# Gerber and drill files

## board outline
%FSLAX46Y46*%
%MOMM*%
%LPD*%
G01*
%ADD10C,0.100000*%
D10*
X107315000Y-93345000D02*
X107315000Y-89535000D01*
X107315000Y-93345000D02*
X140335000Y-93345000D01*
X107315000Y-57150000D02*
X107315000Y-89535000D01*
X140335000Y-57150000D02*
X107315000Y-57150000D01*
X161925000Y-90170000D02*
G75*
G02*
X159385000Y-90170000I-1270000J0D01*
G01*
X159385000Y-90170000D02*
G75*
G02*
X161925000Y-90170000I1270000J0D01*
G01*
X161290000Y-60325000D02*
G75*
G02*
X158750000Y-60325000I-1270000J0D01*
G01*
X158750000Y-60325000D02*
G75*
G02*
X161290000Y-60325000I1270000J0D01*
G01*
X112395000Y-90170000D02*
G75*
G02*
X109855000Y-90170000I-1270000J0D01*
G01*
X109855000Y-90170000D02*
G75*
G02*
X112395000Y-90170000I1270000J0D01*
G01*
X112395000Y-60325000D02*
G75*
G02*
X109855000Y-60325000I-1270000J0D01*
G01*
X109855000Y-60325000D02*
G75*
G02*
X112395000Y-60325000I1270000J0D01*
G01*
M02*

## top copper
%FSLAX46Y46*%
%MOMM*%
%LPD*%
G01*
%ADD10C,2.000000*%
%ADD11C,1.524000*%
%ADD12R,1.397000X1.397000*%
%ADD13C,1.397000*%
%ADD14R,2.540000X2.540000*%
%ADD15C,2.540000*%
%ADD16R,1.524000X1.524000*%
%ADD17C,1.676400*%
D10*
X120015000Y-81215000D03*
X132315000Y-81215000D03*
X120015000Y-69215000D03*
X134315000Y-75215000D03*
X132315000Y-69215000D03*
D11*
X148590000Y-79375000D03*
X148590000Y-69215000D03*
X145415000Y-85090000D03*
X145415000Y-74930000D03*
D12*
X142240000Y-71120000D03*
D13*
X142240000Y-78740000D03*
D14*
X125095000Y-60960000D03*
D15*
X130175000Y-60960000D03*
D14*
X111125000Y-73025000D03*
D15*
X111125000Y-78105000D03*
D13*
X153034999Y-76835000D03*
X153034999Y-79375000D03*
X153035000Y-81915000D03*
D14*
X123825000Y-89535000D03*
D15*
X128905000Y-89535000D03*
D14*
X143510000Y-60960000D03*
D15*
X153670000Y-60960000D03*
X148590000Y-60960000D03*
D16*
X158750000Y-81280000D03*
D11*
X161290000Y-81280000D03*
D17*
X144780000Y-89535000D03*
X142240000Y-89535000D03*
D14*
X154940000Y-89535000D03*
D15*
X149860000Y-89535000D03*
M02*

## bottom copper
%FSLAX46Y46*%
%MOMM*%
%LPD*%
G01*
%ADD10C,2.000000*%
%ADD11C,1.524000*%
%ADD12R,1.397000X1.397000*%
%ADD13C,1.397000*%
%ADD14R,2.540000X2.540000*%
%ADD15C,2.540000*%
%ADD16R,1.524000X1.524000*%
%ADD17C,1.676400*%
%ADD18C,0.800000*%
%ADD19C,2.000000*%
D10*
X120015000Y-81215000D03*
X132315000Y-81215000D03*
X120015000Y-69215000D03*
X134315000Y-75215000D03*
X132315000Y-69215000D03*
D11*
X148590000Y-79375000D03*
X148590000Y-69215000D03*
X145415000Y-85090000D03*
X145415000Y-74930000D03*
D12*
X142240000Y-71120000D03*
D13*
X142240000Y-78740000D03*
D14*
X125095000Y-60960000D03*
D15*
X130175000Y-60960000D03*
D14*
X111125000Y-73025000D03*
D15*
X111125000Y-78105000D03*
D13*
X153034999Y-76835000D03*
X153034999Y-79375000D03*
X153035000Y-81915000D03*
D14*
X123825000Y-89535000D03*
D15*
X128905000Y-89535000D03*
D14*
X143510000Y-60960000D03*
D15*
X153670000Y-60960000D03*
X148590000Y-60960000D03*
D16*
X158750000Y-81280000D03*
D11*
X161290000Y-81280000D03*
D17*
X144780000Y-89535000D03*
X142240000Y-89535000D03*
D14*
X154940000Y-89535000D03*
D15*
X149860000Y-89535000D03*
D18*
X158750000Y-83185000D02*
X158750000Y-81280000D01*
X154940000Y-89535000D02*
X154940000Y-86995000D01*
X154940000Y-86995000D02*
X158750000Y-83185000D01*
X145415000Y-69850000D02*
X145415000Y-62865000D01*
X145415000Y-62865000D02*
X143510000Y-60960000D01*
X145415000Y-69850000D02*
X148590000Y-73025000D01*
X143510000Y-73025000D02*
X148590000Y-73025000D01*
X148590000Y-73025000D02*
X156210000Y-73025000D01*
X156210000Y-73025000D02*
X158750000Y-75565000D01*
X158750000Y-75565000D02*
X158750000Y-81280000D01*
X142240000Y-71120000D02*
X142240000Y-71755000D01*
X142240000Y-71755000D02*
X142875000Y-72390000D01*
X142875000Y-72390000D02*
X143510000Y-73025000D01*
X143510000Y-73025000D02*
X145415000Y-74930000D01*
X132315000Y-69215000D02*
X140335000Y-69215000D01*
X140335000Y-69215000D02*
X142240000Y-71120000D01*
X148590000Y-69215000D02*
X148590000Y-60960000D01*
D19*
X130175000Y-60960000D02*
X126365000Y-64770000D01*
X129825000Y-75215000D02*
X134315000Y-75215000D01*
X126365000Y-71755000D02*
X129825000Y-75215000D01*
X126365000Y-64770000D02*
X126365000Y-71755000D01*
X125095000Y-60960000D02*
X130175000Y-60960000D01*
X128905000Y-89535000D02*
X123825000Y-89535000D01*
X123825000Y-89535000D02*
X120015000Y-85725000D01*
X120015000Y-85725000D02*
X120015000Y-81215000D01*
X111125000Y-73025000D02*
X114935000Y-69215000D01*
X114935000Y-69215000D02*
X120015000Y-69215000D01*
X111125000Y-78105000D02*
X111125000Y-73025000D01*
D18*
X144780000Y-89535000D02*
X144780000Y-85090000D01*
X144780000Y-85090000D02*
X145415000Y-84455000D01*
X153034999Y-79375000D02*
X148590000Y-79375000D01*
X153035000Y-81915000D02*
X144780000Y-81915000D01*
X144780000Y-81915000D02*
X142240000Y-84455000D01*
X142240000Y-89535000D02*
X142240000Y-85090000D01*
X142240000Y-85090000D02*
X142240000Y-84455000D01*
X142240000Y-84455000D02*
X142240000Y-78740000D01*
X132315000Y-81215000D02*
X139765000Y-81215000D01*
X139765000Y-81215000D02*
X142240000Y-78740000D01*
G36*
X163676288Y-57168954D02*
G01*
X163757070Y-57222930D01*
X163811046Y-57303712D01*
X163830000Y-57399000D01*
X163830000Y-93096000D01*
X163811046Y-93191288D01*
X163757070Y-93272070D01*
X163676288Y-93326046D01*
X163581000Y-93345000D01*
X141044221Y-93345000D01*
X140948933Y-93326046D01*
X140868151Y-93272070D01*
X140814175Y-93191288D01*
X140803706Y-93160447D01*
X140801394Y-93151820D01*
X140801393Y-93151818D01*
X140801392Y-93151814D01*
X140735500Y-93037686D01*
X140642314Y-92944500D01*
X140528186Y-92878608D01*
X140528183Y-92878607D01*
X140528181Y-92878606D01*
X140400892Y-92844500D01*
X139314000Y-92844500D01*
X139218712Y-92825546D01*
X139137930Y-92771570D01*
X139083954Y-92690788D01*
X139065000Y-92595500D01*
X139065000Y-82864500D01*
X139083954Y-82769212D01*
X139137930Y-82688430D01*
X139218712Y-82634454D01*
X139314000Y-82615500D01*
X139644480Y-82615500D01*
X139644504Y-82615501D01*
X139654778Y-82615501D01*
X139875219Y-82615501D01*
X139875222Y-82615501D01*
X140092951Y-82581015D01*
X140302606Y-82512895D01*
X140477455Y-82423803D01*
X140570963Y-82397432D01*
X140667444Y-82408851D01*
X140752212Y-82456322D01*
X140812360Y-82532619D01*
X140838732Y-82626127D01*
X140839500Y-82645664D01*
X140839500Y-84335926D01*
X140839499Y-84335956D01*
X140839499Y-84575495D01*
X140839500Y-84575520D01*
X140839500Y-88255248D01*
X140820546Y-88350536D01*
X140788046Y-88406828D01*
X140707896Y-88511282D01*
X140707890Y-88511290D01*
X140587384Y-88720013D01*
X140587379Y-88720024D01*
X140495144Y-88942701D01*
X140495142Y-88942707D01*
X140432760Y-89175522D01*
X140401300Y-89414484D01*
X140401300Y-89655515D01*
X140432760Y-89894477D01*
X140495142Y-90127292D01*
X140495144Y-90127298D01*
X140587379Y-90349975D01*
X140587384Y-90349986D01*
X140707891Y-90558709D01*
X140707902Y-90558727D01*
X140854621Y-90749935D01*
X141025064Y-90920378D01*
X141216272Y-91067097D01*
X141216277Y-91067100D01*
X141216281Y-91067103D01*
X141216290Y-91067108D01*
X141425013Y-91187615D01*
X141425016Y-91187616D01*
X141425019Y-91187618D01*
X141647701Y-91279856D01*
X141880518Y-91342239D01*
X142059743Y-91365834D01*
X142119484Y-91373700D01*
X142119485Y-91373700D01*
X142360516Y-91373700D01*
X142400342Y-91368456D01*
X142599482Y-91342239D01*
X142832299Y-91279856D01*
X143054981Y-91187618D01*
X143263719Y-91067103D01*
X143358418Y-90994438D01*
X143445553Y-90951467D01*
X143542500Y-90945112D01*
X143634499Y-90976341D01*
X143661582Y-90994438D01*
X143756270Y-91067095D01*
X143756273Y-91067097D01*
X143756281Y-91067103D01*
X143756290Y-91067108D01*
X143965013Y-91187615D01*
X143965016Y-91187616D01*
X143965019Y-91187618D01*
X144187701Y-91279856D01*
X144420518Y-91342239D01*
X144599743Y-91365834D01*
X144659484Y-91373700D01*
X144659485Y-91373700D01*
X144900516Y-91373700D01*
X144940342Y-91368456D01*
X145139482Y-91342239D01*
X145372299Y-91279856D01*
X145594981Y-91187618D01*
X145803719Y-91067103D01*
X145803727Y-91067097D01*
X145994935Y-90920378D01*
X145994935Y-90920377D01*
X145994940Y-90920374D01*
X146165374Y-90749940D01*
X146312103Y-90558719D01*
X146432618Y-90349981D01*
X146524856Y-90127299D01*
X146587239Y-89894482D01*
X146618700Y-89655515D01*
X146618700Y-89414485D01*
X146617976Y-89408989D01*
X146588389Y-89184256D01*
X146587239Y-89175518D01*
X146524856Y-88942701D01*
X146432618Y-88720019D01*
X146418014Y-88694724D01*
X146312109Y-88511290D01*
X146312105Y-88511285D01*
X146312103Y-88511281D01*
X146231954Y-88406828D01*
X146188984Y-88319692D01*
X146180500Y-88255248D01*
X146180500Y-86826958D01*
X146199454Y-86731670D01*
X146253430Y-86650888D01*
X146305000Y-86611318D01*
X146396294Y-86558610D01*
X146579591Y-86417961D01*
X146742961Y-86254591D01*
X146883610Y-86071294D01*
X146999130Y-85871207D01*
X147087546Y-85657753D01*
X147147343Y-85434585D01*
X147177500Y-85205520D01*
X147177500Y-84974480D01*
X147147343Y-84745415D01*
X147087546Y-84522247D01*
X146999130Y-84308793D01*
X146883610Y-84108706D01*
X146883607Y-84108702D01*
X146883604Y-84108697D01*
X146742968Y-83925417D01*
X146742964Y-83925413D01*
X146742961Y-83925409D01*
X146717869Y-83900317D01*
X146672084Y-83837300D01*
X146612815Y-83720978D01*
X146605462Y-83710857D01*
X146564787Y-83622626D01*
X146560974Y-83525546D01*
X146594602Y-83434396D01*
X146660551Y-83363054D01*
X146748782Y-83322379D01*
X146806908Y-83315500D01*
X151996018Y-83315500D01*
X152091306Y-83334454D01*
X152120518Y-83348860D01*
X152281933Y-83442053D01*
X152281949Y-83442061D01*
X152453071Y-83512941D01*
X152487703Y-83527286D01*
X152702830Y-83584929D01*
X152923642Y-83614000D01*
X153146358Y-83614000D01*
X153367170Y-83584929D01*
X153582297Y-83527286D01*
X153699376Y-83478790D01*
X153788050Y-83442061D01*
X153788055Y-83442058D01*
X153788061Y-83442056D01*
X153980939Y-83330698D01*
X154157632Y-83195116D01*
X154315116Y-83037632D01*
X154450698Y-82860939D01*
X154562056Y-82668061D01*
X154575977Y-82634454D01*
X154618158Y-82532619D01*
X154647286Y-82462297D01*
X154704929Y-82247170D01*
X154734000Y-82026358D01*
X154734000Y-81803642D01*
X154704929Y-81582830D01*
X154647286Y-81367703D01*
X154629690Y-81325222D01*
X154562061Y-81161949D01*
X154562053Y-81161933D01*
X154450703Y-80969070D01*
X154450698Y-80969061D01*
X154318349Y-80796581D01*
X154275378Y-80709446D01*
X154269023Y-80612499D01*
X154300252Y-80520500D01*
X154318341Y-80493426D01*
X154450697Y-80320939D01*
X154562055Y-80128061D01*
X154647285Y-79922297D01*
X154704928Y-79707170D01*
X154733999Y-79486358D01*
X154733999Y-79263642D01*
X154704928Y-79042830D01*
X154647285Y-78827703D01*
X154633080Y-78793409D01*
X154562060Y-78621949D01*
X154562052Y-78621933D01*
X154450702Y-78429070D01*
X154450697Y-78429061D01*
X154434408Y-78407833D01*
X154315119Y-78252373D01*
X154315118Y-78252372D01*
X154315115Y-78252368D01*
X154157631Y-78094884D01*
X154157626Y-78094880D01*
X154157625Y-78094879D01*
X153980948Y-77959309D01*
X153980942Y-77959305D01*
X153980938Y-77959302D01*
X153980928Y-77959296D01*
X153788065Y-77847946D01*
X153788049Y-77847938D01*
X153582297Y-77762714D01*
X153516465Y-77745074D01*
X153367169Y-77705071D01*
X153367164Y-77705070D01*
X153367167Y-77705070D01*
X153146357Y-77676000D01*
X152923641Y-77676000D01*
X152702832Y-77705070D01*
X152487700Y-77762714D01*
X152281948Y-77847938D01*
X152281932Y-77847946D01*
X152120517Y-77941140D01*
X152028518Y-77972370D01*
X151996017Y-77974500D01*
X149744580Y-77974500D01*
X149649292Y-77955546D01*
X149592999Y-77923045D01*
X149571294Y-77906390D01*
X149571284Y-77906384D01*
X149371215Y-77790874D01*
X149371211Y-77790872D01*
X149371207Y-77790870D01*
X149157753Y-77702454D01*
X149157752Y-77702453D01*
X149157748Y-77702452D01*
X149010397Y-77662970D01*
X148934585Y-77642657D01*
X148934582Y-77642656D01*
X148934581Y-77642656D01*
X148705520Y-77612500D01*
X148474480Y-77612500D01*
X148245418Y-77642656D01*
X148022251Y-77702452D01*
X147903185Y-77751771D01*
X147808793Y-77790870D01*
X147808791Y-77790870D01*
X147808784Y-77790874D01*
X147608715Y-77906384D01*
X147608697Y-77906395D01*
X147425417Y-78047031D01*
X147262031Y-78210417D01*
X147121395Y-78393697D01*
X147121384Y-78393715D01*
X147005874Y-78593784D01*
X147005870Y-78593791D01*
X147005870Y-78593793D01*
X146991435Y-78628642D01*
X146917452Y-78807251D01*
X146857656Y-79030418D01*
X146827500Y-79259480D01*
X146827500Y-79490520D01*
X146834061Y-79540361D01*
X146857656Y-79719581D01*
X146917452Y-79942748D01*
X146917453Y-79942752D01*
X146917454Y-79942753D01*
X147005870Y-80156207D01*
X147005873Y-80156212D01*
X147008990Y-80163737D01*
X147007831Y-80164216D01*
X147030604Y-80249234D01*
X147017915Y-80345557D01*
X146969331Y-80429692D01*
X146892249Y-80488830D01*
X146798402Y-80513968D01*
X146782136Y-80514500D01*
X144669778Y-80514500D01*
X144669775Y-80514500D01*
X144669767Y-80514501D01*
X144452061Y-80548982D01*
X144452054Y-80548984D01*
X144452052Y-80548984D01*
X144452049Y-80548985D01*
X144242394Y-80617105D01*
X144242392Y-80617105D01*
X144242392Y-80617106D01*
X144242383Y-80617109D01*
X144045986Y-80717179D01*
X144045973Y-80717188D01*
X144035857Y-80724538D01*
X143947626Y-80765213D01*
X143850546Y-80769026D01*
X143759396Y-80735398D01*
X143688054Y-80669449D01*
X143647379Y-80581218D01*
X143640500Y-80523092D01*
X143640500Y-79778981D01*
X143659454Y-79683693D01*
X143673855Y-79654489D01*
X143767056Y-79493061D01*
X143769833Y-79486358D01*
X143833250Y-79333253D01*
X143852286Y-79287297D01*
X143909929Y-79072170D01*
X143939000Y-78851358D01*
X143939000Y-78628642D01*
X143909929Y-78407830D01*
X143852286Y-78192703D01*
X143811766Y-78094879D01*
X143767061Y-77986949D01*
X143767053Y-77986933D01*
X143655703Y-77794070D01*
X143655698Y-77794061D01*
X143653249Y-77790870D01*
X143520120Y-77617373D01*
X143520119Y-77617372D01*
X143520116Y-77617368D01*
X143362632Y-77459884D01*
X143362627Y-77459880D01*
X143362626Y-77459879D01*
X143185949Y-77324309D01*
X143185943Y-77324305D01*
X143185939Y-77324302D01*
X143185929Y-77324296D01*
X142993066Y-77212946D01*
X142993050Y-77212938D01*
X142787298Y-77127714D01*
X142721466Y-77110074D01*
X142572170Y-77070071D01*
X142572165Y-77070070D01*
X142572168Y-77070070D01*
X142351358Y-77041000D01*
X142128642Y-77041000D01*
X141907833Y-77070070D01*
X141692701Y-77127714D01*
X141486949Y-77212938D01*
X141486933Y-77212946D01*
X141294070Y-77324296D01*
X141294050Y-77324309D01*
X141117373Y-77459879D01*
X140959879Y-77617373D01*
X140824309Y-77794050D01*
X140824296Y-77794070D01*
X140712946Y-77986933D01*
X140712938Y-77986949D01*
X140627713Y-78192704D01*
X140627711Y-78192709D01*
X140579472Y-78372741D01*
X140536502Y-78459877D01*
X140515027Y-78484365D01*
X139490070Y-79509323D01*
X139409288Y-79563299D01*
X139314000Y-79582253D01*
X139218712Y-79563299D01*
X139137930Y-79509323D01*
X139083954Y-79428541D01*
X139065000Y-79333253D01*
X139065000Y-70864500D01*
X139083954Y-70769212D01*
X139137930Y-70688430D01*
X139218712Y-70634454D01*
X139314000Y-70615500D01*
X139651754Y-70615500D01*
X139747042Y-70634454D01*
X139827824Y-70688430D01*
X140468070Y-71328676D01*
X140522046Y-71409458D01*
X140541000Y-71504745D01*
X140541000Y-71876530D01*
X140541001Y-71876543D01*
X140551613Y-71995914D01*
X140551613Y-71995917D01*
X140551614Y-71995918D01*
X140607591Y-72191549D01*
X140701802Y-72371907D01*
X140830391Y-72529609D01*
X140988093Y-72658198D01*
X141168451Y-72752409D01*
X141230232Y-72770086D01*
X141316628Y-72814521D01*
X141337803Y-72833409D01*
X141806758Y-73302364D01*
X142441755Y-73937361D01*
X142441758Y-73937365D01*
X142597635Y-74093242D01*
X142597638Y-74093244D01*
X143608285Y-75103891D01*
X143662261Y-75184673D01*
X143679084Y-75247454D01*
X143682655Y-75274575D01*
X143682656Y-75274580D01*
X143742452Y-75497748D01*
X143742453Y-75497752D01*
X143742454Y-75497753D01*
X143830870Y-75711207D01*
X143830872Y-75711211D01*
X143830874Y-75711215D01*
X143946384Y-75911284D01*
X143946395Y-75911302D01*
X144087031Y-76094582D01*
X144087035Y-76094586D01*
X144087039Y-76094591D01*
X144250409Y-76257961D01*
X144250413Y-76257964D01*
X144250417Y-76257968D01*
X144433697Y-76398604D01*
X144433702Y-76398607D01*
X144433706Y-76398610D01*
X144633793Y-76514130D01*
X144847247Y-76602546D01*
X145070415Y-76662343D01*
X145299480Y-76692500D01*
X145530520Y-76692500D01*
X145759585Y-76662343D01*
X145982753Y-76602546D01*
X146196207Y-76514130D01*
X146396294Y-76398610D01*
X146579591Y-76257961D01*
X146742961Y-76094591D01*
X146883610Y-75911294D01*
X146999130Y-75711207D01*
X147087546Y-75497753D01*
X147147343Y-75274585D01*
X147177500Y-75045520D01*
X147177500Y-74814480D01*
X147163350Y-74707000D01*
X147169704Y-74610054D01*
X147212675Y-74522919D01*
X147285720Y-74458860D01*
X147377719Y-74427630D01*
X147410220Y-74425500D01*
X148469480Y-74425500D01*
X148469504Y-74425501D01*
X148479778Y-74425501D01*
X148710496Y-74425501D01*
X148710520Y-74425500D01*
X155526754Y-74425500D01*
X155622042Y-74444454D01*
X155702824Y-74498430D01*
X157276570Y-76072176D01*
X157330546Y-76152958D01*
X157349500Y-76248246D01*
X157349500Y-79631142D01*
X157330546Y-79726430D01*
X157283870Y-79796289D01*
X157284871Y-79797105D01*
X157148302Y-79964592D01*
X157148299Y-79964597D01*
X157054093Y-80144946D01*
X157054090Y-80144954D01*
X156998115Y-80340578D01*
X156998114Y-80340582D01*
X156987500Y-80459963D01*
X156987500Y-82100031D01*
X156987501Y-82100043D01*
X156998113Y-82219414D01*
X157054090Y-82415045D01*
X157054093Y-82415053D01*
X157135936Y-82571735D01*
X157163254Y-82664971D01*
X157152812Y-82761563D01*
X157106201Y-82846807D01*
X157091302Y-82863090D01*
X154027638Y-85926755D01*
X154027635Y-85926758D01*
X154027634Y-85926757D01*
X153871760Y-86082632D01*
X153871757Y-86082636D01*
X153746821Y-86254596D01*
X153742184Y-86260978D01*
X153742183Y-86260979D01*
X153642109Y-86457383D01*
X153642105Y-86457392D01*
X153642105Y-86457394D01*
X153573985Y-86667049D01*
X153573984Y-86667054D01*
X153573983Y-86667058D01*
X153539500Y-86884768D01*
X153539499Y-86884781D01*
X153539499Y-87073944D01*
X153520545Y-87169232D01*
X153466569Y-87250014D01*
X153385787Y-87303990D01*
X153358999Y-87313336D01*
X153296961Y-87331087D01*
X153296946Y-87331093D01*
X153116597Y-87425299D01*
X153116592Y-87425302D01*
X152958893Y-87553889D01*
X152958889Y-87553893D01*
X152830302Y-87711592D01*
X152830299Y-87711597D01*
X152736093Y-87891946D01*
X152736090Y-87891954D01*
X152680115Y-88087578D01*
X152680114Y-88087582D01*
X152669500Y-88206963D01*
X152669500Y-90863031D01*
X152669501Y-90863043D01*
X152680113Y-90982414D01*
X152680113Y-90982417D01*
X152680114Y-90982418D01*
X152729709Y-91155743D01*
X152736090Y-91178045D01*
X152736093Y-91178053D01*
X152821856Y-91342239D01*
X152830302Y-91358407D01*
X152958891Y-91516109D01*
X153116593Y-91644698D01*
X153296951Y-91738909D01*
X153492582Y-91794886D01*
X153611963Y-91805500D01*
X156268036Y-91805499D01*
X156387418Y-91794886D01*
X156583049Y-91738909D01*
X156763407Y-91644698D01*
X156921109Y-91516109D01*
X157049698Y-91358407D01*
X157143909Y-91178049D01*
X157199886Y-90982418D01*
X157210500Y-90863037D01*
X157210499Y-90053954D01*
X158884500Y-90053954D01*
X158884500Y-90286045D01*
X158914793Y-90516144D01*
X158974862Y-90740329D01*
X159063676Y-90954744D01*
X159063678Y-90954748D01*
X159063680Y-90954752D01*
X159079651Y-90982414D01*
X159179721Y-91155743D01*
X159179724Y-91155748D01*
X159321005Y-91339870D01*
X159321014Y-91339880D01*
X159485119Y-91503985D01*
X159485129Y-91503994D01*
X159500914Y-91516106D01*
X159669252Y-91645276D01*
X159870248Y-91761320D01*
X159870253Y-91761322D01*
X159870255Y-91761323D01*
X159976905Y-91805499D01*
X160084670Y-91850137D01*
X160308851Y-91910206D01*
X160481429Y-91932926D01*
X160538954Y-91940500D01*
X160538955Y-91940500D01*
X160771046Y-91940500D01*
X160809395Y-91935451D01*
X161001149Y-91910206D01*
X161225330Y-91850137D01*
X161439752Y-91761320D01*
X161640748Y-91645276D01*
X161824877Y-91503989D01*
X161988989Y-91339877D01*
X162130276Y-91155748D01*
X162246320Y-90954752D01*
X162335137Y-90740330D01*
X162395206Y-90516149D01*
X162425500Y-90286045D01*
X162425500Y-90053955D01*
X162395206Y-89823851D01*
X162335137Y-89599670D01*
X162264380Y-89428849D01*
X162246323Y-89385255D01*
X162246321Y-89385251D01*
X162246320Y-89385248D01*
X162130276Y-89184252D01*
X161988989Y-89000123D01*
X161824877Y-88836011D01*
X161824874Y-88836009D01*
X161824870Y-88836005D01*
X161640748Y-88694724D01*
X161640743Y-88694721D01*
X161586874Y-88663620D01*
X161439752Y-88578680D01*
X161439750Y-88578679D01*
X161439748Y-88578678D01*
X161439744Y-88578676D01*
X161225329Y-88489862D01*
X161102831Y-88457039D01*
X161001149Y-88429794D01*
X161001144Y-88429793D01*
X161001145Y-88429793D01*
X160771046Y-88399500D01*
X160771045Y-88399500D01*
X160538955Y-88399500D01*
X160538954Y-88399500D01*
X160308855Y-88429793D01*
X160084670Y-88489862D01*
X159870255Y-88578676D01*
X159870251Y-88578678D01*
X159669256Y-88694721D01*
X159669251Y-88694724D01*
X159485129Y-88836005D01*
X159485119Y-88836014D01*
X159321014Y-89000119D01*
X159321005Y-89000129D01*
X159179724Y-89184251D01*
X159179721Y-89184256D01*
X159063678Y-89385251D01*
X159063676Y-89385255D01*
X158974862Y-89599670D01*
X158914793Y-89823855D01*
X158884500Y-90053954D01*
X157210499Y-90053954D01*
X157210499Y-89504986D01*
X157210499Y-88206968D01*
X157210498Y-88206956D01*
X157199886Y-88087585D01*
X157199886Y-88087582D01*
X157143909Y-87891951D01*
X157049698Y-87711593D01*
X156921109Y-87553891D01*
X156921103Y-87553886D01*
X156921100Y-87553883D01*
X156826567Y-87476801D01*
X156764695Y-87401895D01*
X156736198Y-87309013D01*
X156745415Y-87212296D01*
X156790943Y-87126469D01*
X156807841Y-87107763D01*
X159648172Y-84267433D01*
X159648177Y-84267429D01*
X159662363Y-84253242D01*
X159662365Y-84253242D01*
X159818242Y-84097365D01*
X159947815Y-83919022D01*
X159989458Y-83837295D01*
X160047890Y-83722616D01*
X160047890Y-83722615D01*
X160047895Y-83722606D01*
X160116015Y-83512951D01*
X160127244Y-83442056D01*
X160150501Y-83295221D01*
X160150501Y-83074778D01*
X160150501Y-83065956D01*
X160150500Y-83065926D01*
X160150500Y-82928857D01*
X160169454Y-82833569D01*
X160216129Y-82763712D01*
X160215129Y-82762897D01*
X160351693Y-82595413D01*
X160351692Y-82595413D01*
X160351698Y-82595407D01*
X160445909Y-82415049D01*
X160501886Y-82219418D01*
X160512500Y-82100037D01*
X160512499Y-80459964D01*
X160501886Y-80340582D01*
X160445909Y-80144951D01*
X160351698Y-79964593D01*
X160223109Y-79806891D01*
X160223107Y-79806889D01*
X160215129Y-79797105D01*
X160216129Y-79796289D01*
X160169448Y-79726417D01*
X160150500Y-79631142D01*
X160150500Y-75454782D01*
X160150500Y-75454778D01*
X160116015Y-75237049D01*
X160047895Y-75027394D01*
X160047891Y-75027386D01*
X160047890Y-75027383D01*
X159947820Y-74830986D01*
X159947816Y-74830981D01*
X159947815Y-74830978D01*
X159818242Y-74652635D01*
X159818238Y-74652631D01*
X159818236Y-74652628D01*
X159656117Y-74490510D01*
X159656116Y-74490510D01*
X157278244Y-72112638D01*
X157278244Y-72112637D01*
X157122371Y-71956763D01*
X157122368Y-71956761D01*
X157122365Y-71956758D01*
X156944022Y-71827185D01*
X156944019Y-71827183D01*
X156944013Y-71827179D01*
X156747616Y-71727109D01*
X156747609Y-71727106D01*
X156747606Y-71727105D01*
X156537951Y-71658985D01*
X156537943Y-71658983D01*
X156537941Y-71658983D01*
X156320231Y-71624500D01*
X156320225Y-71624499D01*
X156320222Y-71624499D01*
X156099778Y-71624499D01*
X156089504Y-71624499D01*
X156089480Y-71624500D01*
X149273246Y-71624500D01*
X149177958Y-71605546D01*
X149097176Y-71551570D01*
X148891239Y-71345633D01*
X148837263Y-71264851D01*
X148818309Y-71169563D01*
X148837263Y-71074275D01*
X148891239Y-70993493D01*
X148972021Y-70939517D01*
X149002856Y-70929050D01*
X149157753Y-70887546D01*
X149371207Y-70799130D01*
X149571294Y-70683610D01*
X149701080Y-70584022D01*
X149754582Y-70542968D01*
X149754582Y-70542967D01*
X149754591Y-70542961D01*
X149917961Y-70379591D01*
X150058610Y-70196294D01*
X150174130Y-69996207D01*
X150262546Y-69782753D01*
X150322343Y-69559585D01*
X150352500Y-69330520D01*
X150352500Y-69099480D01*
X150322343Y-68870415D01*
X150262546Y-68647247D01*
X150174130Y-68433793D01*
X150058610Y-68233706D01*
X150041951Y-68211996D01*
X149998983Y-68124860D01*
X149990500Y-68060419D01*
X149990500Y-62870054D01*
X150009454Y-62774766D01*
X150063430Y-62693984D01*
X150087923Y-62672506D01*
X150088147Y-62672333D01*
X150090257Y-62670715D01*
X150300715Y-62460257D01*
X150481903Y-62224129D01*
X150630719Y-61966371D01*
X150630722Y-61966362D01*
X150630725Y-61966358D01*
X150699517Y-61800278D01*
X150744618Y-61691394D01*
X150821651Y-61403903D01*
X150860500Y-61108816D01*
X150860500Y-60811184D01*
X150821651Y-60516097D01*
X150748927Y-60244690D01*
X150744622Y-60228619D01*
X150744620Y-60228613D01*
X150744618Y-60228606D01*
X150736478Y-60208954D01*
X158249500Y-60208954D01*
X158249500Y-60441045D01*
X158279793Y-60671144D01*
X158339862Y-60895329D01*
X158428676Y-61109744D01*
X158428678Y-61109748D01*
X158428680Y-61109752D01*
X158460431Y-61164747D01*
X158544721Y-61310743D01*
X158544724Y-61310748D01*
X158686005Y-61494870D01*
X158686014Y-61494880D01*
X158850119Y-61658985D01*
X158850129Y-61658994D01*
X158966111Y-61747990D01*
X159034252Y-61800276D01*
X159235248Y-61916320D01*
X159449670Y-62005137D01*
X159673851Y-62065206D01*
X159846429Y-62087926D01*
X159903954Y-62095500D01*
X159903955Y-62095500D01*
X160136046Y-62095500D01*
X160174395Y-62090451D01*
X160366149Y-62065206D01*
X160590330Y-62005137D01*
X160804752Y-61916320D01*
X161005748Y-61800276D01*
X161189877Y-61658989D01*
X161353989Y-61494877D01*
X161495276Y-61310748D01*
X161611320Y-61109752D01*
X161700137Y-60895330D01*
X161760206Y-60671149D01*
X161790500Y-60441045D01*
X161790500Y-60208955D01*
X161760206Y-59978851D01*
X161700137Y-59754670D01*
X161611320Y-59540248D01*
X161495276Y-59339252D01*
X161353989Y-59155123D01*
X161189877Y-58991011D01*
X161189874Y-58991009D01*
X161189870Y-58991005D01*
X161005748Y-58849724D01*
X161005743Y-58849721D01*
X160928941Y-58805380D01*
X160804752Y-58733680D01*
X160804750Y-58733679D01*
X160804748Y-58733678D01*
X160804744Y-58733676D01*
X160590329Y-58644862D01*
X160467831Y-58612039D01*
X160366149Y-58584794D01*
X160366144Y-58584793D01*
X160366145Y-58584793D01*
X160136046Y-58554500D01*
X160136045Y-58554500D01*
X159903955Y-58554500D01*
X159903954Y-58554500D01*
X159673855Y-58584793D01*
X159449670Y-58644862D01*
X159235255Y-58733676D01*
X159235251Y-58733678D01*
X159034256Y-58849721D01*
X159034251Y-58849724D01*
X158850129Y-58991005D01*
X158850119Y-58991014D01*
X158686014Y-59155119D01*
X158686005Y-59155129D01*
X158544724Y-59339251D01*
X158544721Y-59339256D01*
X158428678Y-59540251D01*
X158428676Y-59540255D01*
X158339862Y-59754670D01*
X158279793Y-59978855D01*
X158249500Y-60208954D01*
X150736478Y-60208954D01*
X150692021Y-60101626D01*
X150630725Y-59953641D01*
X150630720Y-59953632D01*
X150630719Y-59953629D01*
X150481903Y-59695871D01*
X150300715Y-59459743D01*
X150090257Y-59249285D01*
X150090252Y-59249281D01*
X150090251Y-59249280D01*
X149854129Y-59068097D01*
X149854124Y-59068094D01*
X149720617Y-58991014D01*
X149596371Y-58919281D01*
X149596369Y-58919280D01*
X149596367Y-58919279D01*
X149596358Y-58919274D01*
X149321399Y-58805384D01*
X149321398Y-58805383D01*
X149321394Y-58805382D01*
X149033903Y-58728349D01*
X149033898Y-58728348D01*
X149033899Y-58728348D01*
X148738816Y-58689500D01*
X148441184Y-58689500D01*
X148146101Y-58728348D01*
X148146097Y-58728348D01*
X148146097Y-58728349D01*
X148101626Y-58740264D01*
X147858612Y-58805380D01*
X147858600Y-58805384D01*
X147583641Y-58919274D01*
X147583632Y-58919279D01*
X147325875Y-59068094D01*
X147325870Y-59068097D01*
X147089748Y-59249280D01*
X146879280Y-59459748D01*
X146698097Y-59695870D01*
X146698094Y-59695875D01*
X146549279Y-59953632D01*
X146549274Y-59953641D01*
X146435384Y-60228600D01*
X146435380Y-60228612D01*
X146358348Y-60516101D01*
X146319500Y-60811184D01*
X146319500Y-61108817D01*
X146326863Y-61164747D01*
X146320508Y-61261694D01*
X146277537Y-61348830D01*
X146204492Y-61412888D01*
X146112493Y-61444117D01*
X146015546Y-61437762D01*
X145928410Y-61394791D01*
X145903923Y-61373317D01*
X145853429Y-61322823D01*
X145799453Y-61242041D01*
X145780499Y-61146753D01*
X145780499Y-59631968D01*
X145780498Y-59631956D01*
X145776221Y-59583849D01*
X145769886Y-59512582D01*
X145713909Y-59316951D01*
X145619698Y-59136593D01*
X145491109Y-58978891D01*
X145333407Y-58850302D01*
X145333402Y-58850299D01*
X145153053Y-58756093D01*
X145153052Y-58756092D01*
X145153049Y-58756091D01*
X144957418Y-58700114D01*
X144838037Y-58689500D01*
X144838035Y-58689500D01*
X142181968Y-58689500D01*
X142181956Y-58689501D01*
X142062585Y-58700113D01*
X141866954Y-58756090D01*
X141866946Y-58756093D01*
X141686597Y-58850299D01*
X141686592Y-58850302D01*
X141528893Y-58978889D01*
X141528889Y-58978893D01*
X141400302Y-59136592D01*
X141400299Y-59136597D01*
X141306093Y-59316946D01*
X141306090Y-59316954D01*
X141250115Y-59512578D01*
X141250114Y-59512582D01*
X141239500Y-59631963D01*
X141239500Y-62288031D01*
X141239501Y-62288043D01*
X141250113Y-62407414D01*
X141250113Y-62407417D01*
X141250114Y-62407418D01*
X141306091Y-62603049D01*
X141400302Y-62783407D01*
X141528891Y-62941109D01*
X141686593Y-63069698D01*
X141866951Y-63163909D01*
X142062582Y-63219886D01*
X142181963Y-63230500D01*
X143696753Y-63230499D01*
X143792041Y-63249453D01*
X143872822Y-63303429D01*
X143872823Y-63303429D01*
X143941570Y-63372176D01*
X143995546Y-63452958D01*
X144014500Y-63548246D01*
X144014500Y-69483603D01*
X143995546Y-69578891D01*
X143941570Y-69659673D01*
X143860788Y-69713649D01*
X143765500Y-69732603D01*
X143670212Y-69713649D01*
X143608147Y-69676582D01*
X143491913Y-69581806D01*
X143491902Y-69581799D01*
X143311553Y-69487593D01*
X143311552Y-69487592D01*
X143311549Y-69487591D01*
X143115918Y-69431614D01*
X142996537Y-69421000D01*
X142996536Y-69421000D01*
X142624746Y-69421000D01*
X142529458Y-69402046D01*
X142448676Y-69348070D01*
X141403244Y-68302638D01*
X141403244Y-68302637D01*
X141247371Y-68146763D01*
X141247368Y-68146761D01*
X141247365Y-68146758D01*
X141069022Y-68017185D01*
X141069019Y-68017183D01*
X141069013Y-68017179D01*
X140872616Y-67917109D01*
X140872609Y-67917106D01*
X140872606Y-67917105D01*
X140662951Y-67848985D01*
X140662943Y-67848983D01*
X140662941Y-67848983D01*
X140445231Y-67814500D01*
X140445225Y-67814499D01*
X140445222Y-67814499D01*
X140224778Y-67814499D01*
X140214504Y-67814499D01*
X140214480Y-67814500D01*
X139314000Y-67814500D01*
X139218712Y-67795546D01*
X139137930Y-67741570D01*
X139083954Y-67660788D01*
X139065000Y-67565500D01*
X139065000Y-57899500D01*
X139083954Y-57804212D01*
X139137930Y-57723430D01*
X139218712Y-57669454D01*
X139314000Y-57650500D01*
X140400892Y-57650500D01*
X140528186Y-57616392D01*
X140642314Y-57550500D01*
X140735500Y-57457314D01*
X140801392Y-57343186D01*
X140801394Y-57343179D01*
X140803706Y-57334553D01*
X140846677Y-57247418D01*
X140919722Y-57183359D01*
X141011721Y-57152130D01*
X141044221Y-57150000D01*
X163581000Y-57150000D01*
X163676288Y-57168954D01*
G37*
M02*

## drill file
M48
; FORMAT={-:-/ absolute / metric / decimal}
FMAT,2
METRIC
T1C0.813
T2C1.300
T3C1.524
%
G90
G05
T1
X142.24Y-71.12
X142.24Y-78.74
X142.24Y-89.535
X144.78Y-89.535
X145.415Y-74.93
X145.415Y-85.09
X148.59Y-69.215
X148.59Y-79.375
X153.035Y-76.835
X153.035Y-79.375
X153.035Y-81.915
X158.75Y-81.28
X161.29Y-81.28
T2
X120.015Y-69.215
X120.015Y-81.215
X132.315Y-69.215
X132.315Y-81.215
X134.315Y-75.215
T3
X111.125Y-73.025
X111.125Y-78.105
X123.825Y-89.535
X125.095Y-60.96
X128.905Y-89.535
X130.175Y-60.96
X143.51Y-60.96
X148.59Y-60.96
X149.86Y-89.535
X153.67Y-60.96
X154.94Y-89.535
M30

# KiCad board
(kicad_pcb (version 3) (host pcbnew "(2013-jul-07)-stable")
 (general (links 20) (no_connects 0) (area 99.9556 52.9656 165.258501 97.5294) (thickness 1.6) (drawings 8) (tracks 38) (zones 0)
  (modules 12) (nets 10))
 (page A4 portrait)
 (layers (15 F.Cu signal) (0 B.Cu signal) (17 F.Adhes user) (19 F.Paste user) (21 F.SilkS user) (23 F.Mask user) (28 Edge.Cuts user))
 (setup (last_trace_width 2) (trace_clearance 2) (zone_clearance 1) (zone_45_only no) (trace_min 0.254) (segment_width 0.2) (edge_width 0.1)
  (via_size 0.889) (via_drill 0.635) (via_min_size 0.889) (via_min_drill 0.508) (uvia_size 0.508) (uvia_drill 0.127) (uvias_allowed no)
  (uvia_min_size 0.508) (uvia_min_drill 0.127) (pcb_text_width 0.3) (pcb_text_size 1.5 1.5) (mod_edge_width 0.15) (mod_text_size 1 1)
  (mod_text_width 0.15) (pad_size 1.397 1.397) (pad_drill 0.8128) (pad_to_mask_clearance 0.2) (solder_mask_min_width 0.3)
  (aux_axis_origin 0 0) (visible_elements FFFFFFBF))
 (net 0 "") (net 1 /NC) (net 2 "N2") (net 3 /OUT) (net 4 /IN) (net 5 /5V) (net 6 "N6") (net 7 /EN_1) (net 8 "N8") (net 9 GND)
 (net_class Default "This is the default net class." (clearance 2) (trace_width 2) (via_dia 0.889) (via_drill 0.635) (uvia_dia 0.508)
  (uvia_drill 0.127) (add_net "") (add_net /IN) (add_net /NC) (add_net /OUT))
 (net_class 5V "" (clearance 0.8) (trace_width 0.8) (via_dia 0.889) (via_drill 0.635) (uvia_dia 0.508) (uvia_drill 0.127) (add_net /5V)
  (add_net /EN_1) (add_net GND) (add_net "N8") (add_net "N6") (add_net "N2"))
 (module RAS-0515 (layer F.Cu) (at 120.015 69.215)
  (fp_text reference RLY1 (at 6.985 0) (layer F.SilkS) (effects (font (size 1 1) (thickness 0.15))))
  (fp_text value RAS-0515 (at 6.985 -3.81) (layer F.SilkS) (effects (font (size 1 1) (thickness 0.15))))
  (pad 4 thru_hole circle (at 0 12) (size 2 2) (drill 1.3) (layers *.Cu *.Mask F.SilkS) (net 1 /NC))
  (pad 5 thru_hole circle (at 12.3 12) (size 2 2) (drill 1.3) (layers *.Cu *.Mask F.SilkS) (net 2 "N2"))
  (pad 3 thru_hole circle (at 0 0) (size 2 2) (drill 1.3) (layers *.Cu *.Mask F.SilkS) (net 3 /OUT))
  (pad 1 thru_hole circle (at 14.3 6) (size 2 2) (drill 1.3) (layers *.Cu *.Mask F.SilkS) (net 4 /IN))
  (pad 2 thru_hole circle (at 12.3 0) (size 2 2) (drill 1.3) (layers *.Cu *.Mask F.SilkS) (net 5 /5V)))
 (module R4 (layer F.Cu) (at 148.59 74.295 90) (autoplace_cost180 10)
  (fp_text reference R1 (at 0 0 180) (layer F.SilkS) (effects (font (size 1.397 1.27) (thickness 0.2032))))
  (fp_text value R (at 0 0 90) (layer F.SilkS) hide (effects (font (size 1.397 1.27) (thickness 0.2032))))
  (pad 1 thru_hole circle (at -5.08 0 90) (size 1.524 1.524) (drill 0.8128) (layers *.Cu *.Mask F.SilkS) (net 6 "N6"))
  (pad 2 thru_hole circle (at 5.08 0 90) (size 1.524 1.524) (drill 0.8128) (layers *.Cu *.Mask F.SilkS) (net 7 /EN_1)))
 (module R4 (layer F.Cu) (at 145.415 80.01 90) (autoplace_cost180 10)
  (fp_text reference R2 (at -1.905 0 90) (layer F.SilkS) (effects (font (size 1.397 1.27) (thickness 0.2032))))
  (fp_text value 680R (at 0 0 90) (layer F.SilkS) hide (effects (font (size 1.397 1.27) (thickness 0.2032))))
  (pad 1 thru_hole circle (at -5.08 0 90) (size 1.524 1.524) (drill 0.8128) (layers *.Cu *.Mask F.SilkS) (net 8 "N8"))
  (pad 2 thru_hole circle (at 5.08 0 90) (size 1.524 1.524) (drill 0.8128) (layers *.Cu *.Mask F.SilkS) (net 5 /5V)))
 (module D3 (layer F.Cu) (at 142.24 74.93 90)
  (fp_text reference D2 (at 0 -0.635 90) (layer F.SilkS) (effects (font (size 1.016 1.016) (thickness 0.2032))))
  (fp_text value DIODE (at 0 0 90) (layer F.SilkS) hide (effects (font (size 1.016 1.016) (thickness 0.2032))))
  (pad 2 thru_hole rect (at 3.81 0 90) (size 1.397 1.397) (drill 0.8128) (layers *.Cu *.Mask F.SilkS) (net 5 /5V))
  (pad 1 thru_hole circle (at -3.81 0 90) (size 1.397 1.397) (drill 0.8128) (layers *.Cu *.Mask F.SilkS) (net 2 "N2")))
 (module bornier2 (layer F.Cu) (at 127.635 60.96)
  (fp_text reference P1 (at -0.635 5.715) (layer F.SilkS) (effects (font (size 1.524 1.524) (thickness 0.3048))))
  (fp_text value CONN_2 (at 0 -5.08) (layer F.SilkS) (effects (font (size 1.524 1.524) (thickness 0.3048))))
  (pad 1 thru_hole rect (at -2.54 0) (size 2.54 2.54) (drill 1.524) (layers *.Cu *.Mask F.SilkS) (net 4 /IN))
  (pad 2 thru_hole circle (at 2.54 0) (size 2.54 2.54) (drill 1.524) (layers *.Cu *.Mask F.SilkS) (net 4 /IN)))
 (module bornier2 (layer F.Cu) (at 111.125 75.565 270)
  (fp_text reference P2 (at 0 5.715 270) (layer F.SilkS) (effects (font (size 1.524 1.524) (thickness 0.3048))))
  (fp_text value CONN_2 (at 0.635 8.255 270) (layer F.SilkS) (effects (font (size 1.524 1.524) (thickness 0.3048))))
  (pad 1 thru_hole rect (at -2.54 0 270) (size 2.54 2.54) (drill 1.524) (layers *.Cu *.Mask F.SilkS) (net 3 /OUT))
  (pad 2 thru_hole circle (at 2.54 0 270) (size 2.54 2.54) (drill 1.524) (layers *.Cu *.Mask F.SilkS) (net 3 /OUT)))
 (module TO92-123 (layer F.Cu) (at 154.305 79.375 45)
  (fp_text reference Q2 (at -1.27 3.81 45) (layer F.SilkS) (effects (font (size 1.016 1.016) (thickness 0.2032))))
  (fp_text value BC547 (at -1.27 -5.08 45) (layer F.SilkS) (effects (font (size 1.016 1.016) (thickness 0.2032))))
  (pad 3 thru_hole circle (at 0.898025 -2.694077 45) (size 1.397 1.397) (drill 0.8128) (layers *.Cu *.Mask F.SilkS) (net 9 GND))
  (pad 2 thru_hole circle (at -0.898026 -0.898026 45) (size 1.397 1.397) (drill 0.8128) (layers *.Cu *.Mask F.SilkS) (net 6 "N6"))
  (pad 1 thru_hole circle (at -2.694077 0.898026 45) (size 1.397 1.397) (drill 0.8128) (layers *.Cu *.Mask F.SilkS) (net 2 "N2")))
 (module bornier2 (layer F.Cu) (at 126.365 89.535)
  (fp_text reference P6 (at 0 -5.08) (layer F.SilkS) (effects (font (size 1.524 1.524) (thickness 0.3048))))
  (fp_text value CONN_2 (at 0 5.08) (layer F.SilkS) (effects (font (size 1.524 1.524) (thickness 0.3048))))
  (pad 1 thru_hole rect (at -2.54 0) (size 2.54 2.54) (drill 1.524) (layers *.Cu *.Mask F.SilkS) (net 1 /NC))
  (pad 2 thru_hole circle (at 2.54 0) (size 2.54 2.54) (drill 1.524) (layers *.Cu *.Mask F.SilkS) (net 1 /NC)))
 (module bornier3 (layer F.Cu) (at 148.59 60.96)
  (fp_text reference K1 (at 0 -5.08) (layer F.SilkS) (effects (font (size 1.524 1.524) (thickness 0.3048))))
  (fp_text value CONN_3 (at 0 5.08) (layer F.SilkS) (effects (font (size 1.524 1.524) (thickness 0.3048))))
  (pad 1 thru_hole rect (at -5.08 0) (size 2.54 2.54) (drill 1.524) (layers *.Cu *.Mask F.SilkS) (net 5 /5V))
  (pad 2 thru_hole circle (at 5.08 0) (size 2.54 2.54) (drill 1.524) (layers *.Cu *.Mask F.SilkS) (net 9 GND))
  (pad 3 thru_hole circle (at 0 0) (size 2.54 2.54) (drill 1.524) (layers *.Cu *.Mask F.SilkS) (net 7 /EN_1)))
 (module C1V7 (layer F.Cu) (at 160.02 81.28)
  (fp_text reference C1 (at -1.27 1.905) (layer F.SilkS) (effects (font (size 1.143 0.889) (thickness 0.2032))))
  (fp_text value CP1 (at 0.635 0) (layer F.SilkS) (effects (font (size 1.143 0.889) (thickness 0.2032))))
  (pad 1 thru_hole rect (at -1.27 0) (size 1.524 1.524) (drill 0.8128) (layers *.Cu *.Mask F.SilkS) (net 5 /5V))
  (pad 2 thru_hole circle (at 1.27 0) (size 1.524 1.524) (drill 0.8128) (layers *.Cu *.Mask F.SilkS) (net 9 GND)))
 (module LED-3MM (layer F.Cu) (at 143.51 89.535 180)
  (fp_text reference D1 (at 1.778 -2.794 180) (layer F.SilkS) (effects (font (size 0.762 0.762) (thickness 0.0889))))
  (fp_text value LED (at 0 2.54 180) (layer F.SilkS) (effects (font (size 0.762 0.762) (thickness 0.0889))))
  (pad 1 thru_hole circle (at -1.27 0 180) (size 1.6764 1.6764) (drill 0.8128) (layers *.Cu *.Mask F.SilkS) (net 8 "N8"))
  (pad 2 thru_hole circle (at 1.27 0 180) (size 1.6764 1.6764) (drill 0.8128) (layers *.Cu *.Mask F.SilkS) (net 2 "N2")))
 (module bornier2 (layer F.Cu) (at 152.4 89.535 180)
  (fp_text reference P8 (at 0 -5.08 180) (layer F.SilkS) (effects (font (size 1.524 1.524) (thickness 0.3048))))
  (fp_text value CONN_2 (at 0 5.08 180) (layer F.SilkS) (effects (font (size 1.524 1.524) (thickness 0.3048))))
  (pad 1 thru_hole rect (at -2.54 0 180) (size 2.54 2.54) (drill 1.524) (layers *.Cu *.Mask F.SilkS) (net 5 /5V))
  (pad 2 thru_hole circle (at 2.54 0 180) (size 2.54 2.54) (drill 1.524) (layers *.Cu *.Mask F.SilkS) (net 9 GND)))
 (gr_line (start 107.315 93.345) (end 107.315 89.535) (angle 90) (layer Edge.Cuts) (width 0.1))
 (gr_line (start 107.315 93.345) (end 140.335 93.345) (angle 90) (layer Edge.Cuts) (width 0.1))
 (gr_line (start 107.315 57.15) (end 107.315 89.535) (angle 90) (layer Edge.Cuts) (width 0.1))
 (gr_line (start 140.335 57.15) (end 107.315 57.15) (angle 90) (layer Edge.Cuts) (width 0.1))
 (gr_circle (center 160.655 90.17) (end 161.925 90.17) (layer Edge.Cuts) (width 0.1))
 (gr_circle (center 160.02 60.325) (end 161.29 60.325) (layer Edge.Cuts) (width 0.1))
 (gr_circle (center 111.125 90.17) (end 112.395 90.17) (layer Edge.Cuts) (width 0.1))
 (gr_circle (center 111.125 60.325) (end 112.395 60.325) (layer Edge.Cuts) (width 0.1))
 (segment (start 158.75 83.185) (end 158.75 81.28) (width 0.8) (layer B.Cu) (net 5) (status 800000))
 (segment (start 154.94 89.535) (end 154.94 86.995) (width 0.8) (layer B.Cu) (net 5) (status 400000))
 (segment (start 154.94 86.995) (end 158.75 83.185) (width 0.8) (layer B.Cu) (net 5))
 (segment (start 145.415 69.85) (end 145.415 62.865) (width 0.8) (layer B.Cu) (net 5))
 (segment (start 145.415 62.865) (end 143.51 60.96) (width 0.8) (layer B.Cu) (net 5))
 (segment (start 145.415 69.85) (end 148.59 73.025) (width 0.8) (layer B.Cu) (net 5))
 (segment (start 143.51 73.025) (end 148.59 73.025) (width 0.8) (layer B.Cu) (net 5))
 (segment (start 148.59 73.025) (end 156.21 73.025) (width 0.8) (layer B.Cu) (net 5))
 (segment (start 156.21 73.025) (end 158.75 75.565) (width 0.8) (layer B.Cu) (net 5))
 (segment (start 158.75 75.565) (end 158.75 81.28) (width 0.8) (layer B.Cu) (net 5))
 (segment (start 142.24 71.12) (end 142.24 71.755) (width 0.8) (layer B.Cu) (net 5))
 (segment (start 142.24 71.755) (end 142.875 72.39) (width 0.8) (layer B.Cu) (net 5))
 (segment (start 142.875 72.39) (end 143.51 73.025) (width 0.8) (layer B.Cu) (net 5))
 (segment (start 143.51 73.025) (end 145.415 74.93) (width 0.8) (layer B.Cu) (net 5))
 (segment (start 132.315 69.215) (end 140.335 69.215) (width 0.8) (layer B.Cu) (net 5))
 (segment (start 140.335 69.215) (end 142.24 71.12) (width 0.8) (layer B.Cu) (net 5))
 (segment (start 148.59 69.215) (end 148.59 60.96) (width 0.8) (layer B.Cu) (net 7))
 (segment (start 130.175 60.96) (end 126.365 64.77) (width 2) (layer B.Cu) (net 4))
 (segment (start 129.825 75.215) (end 134.315 75.215) (width 2) (layer B.Cu) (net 4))
 (segment (start 126.365 71.755) (end 129.825 75.215) (width 2) (layer B.Cu) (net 4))
 (segment (start 126.365 64.77) (end 126.365 71.755) (width 2) (layer B.Cu) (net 4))
 (segment (start 125.095 60.96) (end 130.175 60.96) (width 2) (layer B.Cu) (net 4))
 (segment (start 128.905 89.535) (end 123.825 89.535) (width 2) (layer B.Cu) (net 1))
 (segment (start 123.825 89.535) (end 120.015 85.725) (width 2) (layer B.Cu) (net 1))
 (segment (start 120.015 85.725) (end 120.015 81.215) (width 2) (layer B.Cu) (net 1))
 (segment (start 111.125 73.025) (end 114.935 69.215) (width 2) (layer B.Cu) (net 3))
 (segment (start 114.935 69.215) (end 120.015 69.215) (width 2) (layer B.Cu) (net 3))
 (segment (start 111.125 78.105) (end 111.125 73.025) (width 2) (layer B.Cu) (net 3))
 (segment (start 144.78 89.535) (end 144.78 85.09) (width 0.8) (layer B.Cu) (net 8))
 (segment (start 144.78 85.09) (end 145.415 84.455) (width 0.8) (layer B.Cu) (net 8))
 (segment (start 153.034999 79.375) (end 148.59 79.375) (width 0.8) (layer B.Cu) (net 6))
 (segment (start 153.035 81.915) (end 144.78 81.915) (width 0.8) (layer B.Cu) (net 2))
 (segment (start 144.78 81.915) (end 142.24 84.455) (width 0.8) (layer B.Cu) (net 2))
 (segment (start 142.24 89.535) (end 142.24 85.09) (width 0.8) (layer B.Cu) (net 2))
 (segment (start 142.24 85.09) (end 142.24 84.455) (width 0.8) (layer B.Cu) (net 2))
 (segment (start 142.24 84.455) (end 142.24 78.74) (width 0.8) (layer B.Cu) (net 2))
 (segment (start 132.315 81.215) (end 139.765 81.215) (width 0.8) (layer B.Cu) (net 2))
 (segment (start 139.765 81.215) (end 142.24 78.74) (width 0.8) (layer B.Cu) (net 2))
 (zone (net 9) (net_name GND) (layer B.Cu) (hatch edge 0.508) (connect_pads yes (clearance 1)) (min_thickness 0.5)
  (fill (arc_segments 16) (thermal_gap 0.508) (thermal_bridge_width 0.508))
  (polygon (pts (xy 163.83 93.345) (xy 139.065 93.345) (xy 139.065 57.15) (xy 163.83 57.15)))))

